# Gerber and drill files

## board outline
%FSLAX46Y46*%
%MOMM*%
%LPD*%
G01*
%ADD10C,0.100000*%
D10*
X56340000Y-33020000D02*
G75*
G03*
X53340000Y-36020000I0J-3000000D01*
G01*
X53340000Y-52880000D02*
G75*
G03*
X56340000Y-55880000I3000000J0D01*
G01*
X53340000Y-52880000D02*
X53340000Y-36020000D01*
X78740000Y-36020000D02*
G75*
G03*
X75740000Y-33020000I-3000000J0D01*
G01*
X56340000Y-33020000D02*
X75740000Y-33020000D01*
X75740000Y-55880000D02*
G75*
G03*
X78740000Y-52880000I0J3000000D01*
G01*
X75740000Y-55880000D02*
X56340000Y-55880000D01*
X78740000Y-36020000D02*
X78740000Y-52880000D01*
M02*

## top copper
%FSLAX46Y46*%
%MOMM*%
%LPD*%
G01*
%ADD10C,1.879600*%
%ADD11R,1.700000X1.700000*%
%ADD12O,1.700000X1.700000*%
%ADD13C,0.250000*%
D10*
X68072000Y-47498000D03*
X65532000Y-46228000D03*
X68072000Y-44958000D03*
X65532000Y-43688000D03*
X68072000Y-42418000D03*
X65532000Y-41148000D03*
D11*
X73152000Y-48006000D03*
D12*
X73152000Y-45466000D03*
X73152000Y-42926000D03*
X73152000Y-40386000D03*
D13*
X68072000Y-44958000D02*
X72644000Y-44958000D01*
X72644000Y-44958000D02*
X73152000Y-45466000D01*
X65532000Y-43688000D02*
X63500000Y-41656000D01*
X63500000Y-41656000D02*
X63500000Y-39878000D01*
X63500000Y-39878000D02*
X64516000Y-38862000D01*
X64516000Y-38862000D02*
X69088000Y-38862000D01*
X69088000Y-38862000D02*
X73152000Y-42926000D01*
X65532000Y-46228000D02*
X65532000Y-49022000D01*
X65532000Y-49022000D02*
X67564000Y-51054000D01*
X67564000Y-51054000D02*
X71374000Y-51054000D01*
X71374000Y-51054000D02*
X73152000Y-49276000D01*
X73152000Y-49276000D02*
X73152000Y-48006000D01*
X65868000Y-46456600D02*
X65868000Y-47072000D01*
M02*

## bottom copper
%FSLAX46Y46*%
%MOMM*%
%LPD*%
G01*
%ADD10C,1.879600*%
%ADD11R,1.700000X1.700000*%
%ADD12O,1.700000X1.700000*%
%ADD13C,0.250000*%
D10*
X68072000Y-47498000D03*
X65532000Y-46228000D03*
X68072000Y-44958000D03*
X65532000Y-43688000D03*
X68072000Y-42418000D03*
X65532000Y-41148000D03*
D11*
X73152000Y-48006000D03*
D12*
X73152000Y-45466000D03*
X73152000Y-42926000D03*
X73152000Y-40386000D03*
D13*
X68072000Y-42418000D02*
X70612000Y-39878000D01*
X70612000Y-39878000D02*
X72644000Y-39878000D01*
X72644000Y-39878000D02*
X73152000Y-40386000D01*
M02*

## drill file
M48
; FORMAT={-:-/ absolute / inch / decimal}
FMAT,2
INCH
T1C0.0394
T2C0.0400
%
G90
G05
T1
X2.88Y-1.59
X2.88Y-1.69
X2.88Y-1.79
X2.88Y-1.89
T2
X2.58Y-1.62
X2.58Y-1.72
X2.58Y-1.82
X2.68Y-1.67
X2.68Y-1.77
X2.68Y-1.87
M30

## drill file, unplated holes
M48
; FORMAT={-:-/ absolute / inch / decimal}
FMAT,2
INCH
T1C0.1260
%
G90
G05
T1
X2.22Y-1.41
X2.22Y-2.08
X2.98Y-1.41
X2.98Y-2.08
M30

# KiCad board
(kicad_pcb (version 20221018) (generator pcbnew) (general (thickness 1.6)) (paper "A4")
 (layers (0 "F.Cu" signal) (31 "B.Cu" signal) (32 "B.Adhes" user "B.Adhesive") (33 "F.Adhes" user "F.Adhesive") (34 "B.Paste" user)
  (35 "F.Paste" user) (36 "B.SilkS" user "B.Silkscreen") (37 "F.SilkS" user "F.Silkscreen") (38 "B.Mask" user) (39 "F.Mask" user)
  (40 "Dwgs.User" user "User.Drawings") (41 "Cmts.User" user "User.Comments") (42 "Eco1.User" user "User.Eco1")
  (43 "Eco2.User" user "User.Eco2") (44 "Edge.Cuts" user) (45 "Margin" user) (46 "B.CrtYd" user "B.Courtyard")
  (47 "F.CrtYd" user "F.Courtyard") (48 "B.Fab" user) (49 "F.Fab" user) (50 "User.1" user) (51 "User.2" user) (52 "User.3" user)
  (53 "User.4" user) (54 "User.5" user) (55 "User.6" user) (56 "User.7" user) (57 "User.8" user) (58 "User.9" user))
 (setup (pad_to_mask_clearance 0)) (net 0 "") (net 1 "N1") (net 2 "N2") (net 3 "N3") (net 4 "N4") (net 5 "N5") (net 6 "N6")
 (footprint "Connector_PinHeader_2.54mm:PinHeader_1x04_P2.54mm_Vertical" (layer "F.Cu") (at 73.152 48.006 180)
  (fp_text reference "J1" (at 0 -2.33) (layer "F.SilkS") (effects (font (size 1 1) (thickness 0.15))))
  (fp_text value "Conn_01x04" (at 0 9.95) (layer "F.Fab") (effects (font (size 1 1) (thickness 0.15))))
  (pad "1" thru_hole rect (at 0 0 180) (size 1.7 1.7) (drill 1) (layers "*.Cu" "*.Mask") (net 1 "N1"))
  (pad "2" thru_hole oval (at 0 2.54 180) (size 1.7 1.7) (drill 1) (layers "*.Cu" "*.Mask") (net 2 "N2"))
  (pad "3" thru_hole oval (at 0 5.08 180) (size 1.7 1.7) (drill 1) (layers "*.Cu" "*.Mask") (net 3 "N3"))
  (pad "4" thru_hole oval (at 0 7.62 180) (size 1.7 1.7) (drill 1) (layers "*.Cu" "*.Mask") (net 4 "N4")))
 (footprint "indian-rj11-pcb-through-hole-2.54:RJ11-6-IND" (layer "F.Cu") (at 63.672 44.328 -90)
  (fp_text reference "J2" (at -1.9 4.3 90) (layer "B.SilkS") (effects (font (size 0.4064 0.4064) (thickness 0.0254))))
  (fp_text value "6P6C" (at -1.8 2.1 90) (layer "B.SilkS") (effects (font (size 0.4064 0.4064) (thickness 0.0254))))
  (pad "1" thru_hole circle (at 3.17 -4.4 90) (size 1.8796 1.8796) (drill 1.016) (layers "F&B.Cu" "F.Paste" "F.SilkS" "F.Mask") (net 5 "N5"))
  (pad "2" thru_hole circle (at 1.9 -1.86 90) (size 1.8796 1.8796) (drill 1.016) (layers "F&B.Cu" "F.Paste" "F.SilkS" "F.Mask") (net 1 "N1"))
  (pad "3" thru_hole circle (at 0.63 -4.4 90) (size 1.8796 1.8796) (drill 1.016) (layers "F&B.Cu" "F.Paste" "F.SilkS" "F.Mask") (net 2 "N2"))
  (pad "4" thru_hole circle (at -0.64 -1.86 90) (size 1.8796 1.8796) (drill 1.016) (layers "F&B.Cu" "F.Paste" "F.SilkS" "F.Mask")
   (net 3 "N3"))
  (pad "5" thru_hole circle (at -1.91 -4.4 90) (size 1.8796 1.8796) (drill 1.016) (layers "F&B.Cu" "F.Paste" "F.SilkS" "F.Mask")
   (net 4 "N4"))
  (pad "6" thru_hole circle (at -3.18 -1.86 90) (size 1.8796 1.8796) (drill 1.016) (layers "F&B.Cu" "F.Paste" "F.SilkS" "F.Mask")
   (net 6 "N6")))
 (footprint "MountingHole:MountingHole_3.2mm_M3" (layer "F.Cu") (at 56.388 52.832)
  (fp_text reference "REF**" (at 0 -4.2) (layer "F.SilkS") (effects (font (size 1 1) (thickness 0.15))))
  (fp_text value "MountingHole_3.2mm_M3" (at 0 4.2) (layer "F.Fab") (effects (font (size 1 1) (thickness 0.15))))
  (pad "" np_thru_hole circle (at 0 0) (size 3.2 3.2) (drill 3.2) (layers "*.Cu" "*.Mask")))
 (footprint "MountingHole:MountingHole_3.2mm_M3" (layer "F.Cu") (at 75.692 52.832)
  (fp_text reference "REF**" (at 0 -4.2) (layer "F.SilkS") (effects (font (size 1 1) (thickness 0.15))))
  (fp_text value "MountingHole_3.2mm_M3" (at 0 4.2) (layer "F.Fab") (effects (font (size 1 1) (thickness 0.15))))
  (pad "" np_thru_hole circle (at 0 0) (size 3.2 3.2) (drill 3.2) (layers "*.Cu" "*.Mask")))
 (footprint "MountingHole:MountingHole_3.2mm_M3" (layer "F.Cu") (at 75.692 35.814)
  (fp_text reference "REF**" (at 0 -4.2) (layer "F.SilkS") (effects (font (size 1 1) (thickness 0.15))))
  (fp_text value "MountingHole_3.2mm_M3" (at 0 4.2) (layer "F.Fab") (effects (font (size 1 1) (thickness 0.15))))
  (pad "" np_thru_hole circle (at 0 0) (size 3.2 3.2) (drill 3.2) (layers "*.Cu" "*.Mask")))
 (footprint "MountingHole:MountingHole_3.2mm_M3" (layer "F.Cu") (at 56.388 35.814)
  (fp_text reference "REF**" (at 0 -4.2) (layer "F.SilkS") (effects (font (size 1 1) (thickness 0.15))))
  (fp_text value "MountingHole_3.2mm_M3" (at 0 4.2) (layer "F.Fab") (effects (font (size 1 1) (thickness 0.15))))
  (pad "" np_thru_hole circle (at 0 0) (size 3.2 3.2) (drill 3.2) (layers "*.Cu" "*.Mask")))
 (gr_arc (start 75.74 33.02) (mid 77.86132 33.89868) (end 78.74 36.02) (stroke (width 0.1) (type default)) (layer "Edge.Cuts"))
 (gr_line (start 53.34 52.88) (end 53.34 36.02) (stroke (width 0.1) (type default)) (layer "Edge.Cuts"))
 (gr_line (start 56.34 33.02) (end 75.74 33.02) (stroke (width 0.1) (type default)) (layer "Edge.Cuts"))
 (gr_arc (start 56.34 55.88) (mid 54.21868 55.00132) (end 53.34 52.88) (stroke (width 0.1) (type default)) (layer "Edge.Cuts"))
 (gr_line (start 78.74 36.02) (end 78.74 52.88) (stroke (width 0.1) (type default)) (layer "Edge.Cuts"))
 (gr_line (start 75.74 55.88) (end 56.34 55.88) (stroke (width 0.1) (type default)) (layer "Edge.Cuts"))
 (gr_arc (start 53.34 36.02) (mid 54.21868 33.89868) (end 56.34 33.02) (stroke (width 0.1) (type default)) (layer "Edge.Cuts"))
 (gr_arc (start 78.74 52.88) (mid 77.86132 55.00132) (end 75.74 55.88) (stroke (width 0.1) (type default)) (layer "Edge.Cuts"))
 (segment (start 73.152 49.276) (end 73.152 48.006) (width 0.25) (layer "F.Cu") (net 1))
 (segment (start 65.868 46.4566) (end 65.868 47.072) (width 0.25) (layer "F.Cu") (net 1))
 (segment (start 65.532 46.228) (end 65.532 49.022) (width 0.25) (layer "F.Cu") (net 1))
 (segment (start 71.374 51.054) (end 73.152 49.276) (width 0.25) (layer "F.Cu") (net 1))
 (segment (start 67.564 51.054) (end 71.374 51.054) (width 0.25) (layer "F.Cu") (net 1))
 (segment (start 65.532 49.022) (end 67.564 51.054) (width 0.25) (layer "F.Cu") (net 1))
 (segment (start 72.644 44.958) (end 73.152 45.466) (width 0.25) (layer "F.Cu") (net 2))
 (segment (start 68.072 44.958) (end 72.644 44.958) (width 0.25) (layer "F.Cu") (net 2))
 (segment (start 63.5 41.656) (end 63.5 39.878) (width 0.25) (layer "F.Cu") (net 3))
 (segment (start 65.532 43.688) (end 63.5 41.656) (width 0.25) (layer "F.Cu") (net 3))
 (segment (start 63.5 39.878) (end 64.516 38.862) (width 0.25) (layer "F.Cu") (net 3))
 (segment (start 69.088 38.862) (end 73.152 42.926) (width 0.25) (layer "F.Cu") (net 3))
 (segment (start 64.516 38.862) (end 69.088 38.862) (width 0.25) (layer "F.Cu") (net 3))
 (segment (start 68.072 42.418) (end 70.612 39.878) (width 0.25) (layer "B.Cu") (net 4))
 (segment (start 70.612 39.878) (end 72.644 39.878) (width 0.25) (layer "B.Cu") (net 4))
 (segment (start 72.644 39.878) (end 73.152 40.386) (width 0.25) (layer "B.Cu") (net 4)))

